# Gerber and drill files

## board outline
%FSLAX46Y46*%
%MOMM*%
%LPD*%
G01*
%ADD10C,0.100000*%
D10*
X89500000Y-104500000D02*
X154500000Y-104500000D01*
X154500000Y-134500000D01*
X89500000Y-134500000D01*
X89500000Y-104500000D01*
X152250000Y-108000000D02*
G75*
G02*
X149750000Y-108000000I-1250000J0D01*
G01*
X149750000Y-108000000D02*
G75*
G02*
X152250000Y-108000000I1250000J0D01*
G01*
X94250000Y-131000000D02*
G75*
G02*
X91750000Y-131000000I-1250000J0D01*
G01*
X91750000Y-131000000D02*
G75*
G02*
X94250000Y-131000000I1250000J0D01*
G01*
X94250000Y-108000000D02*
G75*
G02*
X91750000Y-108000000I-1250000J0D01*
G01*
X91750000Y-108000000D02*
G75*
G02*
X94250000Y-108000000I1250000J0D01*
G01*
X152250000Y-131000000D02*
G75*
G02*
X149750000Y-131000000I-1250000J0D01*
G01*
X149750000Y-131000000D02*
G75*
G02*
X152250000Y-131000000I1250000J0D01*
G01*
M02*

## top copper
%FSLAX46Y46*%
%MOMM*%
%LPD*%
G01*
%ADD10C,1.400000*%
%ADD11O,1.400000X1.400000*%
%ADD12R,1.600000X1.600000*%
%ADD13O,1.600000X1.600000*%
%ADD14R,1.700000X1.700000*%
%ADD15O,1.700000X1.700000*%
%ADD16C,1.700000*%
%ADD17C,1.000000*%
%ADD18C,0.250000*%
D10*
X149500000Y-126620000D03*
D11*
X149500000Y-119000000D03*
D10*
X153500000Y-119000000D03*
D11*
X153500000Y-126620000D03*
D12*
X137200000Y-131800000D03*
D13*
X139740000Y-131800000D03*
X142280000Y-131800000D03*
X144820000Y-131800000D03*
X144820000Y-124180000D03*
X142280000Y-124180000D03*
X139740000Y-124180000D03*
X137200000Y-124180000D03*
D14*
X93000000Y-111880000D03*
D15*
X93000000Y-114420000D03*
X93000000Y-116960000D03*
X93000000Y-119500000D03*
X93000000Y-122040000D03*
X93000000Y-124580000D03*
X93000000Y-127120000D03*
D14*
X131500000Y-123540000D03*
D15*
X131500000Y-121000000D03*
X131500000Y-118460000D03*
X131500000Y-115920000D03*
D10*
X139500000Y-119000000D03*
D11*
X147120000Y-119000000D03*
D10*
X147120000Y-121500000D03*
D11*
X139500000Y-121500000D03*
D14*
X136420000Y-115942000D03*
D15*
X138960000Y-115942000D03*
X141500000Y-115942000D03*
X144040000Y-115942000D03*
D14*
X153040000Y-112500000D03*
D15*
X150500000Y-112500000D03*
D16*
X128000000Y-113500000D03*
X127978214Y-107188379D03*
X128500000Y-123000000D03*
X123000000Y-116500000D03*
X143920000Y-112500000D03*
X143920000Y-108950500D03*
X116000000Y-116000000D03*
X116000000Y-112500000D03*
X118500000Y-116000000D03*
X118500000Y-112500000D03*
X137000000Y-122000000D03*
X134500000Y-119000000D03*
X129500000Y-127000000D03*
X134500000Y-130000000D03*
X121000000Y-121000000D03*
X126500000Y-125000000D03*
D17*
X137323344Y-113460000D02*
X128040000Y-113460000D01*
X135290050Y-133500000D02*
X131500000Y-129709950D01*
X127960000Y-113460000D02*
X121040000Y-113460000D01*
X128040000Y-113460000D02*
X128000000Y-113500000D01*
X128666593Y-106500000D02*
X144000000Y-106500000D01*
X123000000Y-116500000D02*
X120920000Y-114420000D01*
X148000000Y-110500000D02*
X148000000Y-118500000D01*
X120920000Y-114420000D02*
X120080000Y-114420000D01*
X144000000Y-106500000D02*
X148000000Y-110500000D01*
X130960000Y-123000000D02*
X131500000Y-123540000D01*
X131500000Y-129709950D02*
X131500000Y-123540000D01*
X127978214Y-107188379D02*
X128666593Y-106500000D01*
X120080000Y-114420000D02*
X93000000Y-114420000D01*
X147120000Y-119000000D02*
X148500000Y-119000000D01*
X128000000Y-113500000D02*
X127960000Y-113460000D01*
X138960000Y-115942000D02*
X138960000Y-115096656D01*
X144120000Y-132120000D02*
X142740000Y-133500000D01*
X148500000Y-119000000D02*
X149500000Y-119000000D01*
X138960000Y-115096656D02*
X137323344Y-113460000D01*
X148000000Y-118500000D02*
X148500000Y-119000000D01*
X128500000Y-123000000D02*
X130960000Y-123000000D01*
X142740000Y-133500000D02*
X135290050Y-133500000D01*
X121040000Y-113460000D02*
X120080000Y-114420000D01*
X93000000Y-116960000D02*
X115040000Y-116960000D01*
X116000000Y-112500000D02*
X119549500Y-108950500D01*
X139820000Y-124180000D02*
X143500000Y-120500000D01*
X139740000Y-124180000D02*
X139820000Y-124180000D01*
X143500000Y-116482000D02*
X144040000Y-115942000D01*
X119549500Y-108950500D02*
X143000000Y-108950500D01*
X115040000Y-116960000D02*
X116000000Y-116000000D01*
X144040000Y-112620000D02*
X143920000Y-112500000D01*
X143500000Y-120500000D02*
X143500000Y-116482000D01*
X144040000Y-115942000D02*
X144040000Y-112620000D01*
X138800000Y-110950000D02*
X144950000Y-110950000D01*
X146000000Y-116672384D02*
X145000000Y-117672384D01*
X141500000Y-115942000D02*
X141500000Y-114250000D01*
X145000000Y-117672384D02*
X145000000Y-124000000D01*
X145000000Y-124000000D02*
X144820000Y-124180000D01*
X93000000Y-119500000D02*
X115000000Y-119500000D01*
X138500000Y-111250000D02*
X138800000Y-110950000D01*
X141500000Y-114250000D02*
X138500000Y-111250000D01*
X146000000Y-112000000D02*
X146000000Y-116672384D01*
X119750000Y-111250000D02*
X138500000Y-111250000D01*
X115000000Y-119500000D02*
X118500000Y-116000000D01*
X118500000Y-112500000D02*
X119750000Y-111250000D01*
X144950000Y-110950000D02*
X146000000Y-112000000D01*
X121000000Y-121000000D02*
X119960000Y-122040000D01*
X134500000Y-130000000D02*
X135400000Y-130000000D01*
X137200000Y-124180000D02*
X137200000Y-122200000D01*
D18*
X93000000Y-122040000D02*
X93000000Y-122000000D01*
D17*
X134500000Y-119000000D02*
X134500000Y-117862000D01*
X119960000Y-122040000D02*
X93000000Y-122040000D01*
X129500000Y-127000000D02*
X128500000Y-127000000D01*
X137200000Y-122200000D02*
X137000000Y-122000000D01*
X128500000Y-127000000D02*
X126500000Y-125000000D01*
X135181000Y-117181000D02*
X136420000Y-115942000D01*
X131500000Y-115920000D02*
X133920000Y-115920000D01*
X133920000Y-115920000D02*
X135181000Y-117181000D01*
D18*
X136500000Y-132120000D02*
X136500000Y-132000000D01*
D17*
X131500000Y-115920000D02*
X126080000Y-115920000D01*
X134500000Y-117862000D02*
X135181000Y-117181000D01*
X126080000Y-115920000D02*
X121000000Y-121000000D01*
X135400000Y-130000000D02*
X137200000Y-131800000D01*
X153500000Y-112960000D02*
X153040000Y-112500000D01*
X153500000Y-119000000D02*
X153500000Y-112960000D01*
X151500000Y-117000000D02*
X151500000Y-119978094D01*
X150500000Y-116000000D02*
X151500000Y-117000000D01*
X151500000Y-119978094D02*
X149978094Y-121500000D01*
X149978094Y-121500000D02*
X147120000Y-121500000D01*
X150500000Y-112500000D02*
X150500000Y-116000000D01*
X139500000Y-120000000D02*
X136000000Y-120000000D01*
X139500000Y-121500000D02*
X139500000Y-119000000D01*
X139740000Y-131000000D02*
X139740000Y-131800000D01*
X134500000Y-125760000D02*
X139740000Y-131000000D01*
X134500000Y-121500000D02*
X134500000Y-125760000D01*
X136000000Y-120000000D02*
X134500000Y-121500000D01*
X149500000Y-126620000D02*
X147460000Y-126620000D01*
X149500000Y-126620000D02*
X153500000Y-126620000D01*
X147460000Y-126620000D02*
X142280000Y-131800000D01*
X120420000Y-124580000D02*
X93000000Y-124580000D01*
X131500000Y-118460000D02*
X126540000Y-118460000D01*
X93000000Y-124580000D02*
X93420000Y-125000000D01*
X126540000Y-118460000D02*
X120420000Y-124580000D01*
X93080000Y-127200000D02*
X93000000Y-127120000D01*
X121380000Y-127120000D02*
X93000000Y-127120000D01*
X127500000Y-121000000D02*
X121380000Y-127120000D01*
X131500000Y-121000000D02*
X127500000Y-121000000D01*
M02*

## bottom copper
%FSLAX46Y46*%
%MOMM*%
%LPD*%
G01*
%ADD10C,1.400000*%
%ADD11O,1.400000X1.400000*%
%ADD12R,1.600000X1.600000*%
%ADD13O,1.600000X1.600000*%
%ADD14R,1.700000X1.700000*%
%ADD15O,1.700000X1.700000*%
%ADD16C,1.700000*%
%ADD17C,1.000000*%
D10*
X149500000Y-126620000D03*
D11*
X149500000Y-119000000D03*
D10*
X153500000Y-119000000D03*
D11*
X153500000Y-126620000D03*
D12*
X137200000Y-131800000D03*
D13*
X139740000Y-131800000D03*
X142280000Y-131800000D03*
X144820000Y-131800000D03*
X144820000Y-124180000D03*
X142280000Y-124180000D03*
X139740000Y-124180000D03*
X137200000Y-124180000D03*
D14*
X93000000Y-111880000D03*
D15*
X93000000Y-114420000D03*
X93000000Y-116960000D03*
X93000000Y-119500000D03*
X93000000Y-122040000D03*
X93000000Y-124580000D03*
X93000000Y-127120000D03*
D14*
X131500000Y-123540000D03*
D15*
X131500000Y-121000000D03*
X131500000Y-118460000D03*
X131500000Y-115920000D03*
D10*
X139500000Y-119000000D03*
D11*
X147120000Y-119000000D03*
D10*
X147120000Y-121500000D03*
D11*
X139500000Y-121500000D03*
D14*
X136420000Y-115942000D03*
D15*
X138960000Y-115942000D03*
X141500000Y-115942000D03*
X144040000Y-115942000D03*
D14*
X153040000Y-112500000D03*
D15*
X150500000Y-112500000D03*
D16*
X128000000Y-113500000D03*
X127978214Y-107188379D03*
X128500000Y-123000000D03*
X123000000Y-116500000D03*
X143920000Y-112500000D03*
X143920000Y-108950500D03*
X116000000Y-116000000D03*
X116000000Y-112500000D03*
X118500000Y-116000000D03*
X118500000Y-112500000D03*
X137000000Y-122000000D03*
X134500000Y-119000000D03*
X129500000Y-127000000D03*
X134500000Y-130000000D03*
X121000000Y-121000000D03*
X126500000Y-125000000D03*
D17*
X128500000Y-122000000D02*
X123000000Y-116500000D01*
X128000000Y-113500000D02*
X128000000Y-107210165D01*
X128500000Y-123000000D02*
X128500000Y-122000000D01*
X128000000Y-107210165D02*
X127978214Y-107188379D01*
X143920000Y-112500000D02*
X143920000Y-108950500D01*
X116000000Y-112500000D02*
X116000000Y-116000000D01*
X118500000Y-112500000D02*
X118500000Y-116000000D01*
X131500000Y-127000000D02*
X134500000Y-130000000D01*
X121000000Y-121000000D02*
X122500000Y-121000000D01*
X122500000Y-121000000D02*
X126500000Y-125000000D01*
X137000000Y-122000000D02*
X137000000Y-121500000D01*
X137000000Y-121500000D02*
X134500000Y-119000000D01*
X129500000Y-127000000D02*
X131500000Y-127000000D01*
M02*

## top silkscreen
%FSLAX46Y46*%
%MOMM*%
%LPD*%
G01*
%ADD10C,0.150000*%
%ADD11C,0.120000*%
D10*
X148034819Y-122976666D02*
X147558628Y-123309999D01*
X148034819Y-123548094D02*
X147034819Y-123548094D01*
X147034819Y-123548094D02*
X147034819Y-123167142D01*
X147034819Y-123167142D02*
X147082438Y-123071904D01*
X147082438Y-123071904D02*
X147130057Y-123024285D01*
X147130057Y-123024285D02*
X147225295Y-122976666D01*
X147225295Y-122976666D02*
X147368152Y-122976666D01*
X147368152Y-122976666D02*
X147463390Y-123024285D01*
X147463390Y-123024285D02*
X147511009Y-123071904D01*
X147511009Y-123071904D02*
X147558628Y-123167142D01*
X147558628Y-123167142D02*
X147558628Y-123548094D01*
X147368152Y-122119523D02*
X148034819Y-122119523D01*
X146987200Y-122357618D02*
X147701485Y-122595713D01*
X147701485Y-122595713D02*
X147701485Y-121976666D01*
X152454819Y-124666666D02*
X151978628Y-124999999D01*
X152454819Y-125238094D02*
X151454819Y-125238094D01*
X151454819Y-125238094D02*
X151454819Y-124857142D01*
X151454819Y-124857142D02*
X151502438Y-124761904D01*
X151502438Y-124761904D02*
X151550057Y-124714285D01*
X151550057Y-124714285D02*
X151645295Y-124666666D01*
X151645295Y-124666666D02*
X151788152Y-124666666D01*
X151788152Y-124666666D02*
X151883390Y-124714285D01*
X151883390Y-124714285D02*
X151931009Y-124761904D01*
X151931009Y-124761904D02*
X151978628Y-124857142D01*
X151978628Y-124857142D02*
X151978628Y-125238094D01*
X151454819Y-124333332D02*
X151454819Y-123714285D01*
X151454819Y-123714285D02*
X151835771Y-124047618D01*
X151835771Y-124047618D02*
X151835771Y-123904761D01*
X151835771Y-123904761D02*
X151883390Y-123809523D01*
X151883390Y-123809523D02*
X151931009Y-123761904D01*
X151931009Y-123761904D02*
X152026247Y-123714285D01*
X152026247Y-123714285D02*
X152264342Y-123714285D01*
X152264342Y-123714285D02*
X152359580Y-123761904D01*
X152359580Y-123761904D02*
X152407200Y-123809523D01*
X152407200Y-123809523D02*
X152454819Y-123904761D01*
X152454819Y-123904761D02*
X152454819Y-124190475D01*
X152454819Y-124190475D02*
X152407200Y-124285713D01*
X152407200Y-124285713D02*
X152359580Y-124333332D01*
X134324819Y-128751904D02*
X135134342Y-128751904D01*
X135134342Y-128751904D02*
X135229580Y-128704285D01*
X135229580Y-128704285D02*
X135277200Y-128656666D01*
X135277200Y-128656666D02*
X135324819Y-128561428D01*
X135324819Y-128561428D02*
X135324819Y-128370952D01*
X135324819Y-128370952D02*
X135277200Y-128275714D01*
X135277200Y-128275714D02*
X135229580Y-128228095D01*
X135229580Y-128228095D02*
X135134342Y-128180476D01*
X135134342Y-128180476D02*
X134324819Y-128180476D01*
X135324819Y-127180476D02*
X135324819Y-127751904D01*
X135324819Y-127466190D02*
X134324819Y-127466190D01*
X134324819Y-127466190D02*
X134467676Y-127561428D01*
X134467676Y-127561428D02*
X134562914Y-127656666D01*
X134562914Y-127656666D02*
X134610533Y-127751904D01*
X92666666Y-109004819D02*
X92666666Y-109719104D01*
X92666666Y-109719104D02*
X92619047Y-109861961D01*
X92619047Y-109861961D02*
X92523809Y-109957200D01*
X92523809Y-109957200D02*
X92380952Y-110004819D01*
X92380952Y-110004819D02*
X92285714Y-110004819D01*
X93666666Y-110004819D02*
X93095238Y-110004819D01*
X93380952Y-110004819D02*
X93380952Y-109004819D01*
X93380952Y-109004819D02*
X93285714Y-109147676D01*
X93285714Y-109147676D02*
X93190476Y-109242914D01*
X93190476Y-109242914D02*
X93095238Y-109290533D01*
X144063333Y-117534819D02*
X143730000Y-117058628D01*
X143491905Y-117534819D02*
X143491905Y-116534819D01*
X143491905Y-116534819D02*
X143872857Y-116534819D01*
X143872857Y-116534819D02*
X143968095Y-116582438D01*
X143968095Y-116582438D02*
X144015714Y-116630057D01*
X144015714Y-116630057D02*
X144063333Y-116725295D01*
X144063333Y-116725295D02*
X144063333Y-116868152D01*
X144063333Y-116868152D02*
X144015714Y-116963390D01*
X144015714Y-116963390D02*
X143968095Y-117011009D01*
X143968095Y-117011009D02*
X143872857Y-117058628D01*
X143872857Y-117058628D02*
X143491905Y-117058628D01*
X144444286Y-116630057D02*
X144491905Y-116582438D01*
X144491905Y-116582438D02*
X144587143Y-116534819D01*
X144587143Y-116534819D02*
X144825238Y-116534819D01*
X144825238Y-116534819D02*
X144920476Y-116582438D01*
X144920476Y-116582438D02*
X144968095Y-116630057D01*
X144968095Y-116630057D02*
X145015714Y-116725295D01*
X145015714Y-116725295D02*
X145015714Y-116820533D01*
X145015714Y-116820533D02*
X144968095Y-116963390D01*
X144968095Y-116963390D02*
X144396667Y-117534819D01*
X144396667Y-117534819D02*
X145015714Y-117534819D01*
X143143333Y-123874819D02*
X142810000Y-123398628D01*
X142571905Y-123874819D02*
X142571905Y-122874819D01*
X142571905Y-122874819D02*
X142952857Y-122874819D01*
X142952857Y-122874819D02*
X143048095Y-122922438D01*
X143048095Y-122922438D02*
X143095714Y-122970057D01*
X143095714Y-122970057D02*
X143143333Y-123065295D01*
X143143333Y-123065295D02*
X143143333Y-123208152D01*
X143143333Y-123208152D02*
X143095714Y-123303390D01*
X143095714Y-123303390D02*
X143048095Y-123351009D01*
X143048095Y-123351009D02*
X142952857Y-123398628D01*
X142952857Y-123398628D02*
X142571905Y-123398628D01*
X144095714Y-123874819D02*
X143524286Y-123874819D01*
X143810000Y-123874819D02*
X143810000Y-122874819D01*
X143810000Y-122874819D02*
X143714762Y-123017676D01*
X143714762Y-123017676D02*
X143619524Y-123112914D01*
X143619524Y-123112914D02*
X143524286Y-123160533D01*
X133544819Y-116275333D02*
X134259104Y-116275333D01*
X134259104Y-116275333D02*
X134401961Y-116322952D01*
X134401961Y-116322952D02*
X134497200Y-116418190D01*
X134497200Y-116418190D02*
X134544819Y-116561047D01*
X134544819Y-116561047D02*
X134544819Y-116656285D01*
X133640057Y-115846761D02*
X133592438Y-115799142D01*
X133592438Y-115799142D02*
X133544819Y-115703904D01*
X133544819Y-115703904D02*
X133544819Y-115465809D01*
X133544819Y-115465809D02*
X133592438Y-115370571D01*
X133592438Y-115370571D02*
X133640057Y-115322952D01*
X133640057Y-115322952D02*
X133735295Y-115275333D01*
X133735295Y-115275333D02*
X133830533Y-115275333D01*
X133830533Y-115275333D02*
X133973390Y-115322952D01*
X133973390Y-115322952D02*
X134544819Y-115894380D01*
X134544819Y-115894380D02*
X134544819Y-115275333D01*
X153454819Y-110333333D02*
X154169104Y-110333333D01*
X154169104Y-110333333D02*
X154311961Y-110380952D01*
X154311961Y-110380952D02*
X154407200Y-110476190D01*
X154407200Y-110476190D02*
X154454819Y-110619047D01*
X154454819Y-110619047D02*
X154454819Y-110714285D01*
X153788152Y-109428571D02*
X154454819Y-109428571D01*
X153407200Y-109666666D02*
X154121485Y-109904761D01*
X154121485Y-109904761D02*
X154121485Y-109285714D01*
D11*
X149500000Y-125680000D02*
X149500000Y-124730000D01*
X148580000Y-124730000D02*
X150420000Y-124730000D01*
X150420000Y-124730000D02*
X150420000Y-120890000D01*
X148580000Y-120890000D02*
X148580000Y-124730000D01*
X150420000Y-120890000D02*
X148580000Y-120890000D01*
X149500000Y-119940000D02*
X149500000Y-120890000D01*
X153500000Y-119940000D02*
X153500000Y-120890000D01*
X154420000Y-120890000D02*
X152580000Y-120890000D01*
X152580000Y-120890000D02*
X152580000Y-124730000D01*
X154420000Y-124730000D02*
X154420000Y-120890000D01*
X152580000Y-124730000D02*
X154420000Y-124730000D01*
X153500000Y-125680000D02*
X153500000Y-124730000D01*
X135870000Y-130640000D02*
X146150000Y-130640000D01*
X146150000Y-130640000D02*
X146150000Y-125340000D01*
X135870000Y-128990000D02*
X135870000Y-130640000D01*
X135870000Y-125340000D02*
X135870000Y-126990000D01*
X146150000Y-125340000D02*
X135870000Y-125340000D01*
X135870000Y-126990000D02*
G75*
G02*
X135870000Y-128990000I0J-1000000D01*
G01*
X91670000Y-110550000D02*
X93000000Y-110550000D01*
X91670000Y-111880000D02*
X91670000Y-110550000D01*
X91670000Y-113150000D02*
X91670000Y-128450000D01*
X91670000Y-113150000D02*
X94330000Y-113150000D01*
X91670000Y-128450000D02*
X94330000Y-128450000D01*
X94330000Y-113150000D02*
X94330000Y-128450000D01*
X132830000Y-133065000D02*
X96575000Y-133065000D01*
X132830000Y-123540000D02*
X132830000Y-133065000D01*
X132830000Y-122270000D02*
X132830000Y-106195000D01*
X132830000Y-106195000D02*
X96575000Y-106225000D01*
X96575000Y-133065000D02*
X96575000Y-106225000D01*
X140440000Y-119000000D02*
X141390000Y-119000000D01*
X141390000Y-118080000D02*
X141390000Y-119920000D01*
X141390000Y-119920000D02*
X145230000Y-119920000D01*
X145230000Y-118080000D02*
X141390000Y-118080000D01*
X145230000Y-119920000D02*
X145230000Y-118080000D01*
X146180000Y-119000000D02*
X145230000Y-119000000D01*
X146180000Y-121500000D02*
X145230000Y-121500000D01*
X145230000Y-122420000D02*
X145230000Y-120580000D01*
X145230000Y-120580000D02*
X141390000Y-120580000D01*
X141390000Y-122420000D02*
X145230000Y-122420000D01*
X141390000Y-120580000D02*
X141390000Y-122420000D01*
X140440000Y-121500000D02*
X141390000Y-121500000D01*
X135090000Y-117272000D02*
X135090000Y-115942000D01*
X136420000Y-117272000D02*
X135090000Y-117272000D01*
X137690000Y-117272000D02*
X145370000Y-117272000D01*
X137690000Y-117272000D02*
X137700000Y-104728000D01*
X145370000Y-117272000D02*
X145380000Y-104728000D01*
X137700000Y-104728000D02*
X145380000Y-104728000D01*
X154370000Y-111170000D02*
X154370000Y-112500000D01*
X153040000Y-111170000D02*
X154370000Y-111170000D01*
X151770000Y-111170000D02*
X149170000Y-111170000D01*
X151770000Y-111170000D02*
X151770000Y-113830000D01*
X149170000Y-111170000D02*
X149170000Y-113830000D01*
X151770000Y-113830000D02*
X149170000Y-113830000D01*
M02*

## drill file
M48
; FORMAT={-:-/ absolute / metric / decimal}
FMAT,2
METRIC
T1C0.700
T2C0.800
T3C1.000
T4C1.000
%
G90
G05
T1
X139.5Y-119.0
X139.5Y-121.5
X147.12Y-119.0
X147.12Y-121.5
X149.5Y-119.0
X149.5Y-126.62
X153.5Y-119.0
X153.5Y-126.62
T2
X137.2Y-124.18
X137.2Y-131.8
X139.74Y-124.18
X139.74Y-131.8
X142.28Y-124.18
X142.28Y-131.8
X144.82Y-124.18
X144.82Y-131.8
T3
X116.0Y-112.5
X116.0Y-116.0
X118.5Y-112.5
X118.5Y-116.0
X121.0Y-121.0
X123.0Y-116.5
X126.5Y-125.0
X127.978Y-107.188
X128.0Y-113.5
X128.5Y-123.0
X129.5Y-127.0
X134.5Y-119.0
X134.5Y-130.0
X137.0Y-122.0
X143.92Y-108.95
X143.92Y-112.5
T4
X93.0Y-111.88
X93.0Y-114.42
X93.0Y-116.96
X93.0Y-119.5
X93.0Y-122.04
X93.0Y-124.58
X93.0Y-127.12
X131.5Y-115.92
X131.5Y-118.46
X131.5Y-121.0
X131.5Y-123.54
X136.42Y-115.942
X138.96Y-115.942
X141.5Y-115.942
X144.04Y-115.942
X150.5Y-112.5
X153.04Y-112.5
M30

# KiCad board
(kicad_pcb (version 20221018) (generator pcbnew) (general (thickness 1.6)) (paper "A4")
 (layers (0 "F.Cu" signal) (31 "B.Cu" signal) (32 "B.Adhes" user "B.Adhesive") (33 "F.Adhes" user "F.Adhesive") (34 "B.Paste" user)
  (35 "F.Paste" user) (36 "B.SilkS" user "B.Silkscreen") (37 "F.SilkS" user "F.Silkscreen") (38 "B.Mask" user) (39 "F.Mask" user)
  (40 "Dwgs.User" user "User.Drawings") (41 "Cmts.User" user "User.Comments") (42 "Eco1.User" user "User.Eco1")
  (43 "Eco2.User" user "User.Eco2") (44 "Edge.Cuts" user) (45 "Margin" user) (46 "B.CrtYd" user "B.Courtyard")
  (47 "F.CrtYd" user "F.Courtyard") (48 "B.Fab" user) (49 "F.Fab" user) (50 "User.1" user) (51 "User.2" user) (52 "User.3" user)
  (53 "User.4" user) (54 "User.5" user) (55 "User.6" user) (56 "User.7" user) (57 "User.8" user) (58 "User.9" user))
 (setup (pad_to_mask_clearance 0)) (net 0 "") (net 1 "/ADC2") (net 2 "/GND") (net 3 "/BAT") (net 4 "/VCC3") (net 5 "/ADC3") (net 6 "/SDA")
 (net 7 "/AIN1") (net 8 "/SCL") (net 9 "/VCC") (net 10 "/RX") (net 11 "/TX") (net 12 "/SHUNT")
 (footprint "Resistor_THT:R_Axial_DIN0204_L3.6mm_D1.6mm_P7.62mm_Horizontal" (layer "F.Cu") (at 149.5 126.62 90)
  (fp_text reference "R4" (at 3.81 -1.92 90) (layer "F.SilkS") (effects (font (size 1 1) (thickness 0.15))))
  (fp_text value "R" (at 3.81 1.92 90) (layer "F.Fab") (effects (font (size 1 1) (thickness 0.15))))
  (fp_line (start 0.94 0) (end 1.89 0) (stroke (width 0.12) (type solid)) (layer "F.SilkS"))
  (fp_line (start 1.89 -0.92) (end 1.89 0.92) (stroke (width 0.12) (type solid)) (layer "F.SilkS"))
  (fp_line (start 1.89 0.92) (end 5.73 0.92) (stroke (width 0.12) (type solid)) (layer "F.SilkS"))
  (fp_line (start 5.73 -0.92) (end 1.89 -0.92) (stroke (width 0.12) (type solid)) (layer "F.SilkS"))
  (fp_line (start 5.73 0.92) (end 5.73 -0.92) (stroke (width 0.12) (type solid)) (layer "F.SilkS"))
  (fp_line (start 6.68 0) (end 5.73 0) (stroke (width 0.12) (type solid)) (layer "F.SilkS"))
  (pad "1" thru_hole circle (at 0 0 90) (size 1.4 1.4) (drill 0.7) (layers "*.Cu" "*.Mask") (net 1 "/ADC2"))
  (pad "2" thru_hole oval (at 7.62 0 90) (size 1.4 1.4) (drill 0.7) (layers "*.Cu" "*.Mask") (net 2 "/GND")))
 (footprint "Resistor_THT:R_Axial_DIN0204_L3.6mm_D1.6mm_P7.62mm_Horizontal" (layer "F.Cu") (at 153.5 119 -90)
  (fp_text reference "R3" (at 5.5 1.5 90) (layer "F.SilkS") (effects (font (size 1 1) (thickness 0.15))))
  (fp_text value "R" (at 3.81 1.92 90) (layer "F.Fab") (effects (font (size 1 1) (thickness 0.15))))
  (fp_line (start 0.94 0) (end 1.89 0) (stroke (width 0.12) (type solid)) (layer "F.SilkS"))
  (fp_line (start 1.89 -0.92) (end 1.89 0.92) (stroke (width 0.12) (type solid)) (layer "F.SilkS"))
  (fp_line (start 1.89 0.92) (end 5.73 0.92) (stroke (width 0.12) (type solid)) (layer "F.SilkS"))
  (fp_line (start 5.73 -0.92) (end 1.89 -0.92) (stroke (width 0.12) (type solid)) (layer "F.SilkS"))
  (fp_line (start 5.73 0.92) (end 5.73 -0.92) (stroke (width 0.12) (type solid)) (layer "F.SilkS"))
  (fp_line (start 6.68 0) (end 5.73 0) (stroke (width 0.12) (type solid)) (layer "F.SilkS"))
  (pad "1" thru_hole circle (at 0 0 270) (size 1.4 1.4) (drill 0.7) (layers "*.Cu" "*.Mask") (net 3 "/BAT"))
  (pad "2" thru_hole oval (at 7.62 0 270) (size 1.4 1.4) (drill 0.7) (layers "*.Cu" "*.Mask") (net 1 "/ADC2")))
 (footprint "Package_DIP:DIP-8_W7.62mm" (layer "F.Cu") (at 137.2 131.8 90)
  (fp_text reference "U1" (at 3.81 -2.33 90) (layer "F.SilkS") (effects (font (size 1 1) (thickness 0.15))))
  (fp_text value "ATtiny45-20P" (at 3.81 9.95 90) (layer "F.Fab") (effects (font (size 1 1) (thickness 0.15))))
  (fp_line (start 1.16 -1.33) (end 1.16 8.95) (stroke (width 0.12) (type solid)) (layer "F.SilkS"))
  (fp_line (start 1.16 8.95) (end 6.46 8.95) (stroke (width 0.12) (type solid)) (layer "F.SilkS"))
  (fp_line (start 2.81 -1.33) (end 1.16 -1.33) (stroke (width 0.12) (type solid)) (layer "F.SilkS"))
  (fp_line (start 6.46 -1.33) (end 4.81 -1.33) (stroke (width 0.12) (type solid)) (layer "F.SilkS"))
  (fp_line (start 6.46 8.95) (end 6.46 -1.33) (stroke (width 0.12) (type solid)) (layer "F.SilkS"))
  (fp_arc (start 4.81 -1.33) (mid 3.81 -0.33) (end 2.81 -1.33) (stroke (width 0.12) (type solid)) (layer "F.SilkS"))
  (pad "1" thru_hole rect (at 0 0 90) (size 1.6 1.6) (drill 0.8) (layers "*.Cu" "*.Mask") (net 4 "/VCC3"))
  (pad "2" thru_hole oval (at 0 2.54 90) (size 1.6 1.6) (drill 0.8) (layers "*.Cu" "*.Mask") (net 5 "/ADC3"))
  (pad "3" thru_hole oval (at 0 5.08 90) (size 1.6 1.6) (drill 0.8) (layers "*.Cu" "*.Mask") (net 1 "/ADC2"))
  (pad "4" thru_hole oval (at 0 7.62 90) (size 1.6 1.6) (drill 0.8) (layers "*.Cu" "*.Mask") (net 2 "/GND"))
  (pad "5" thru_hole oval (at 7.62 7.62 90) (size 1.6 1.6) (drill 0.8) (layers "*.Cu" "*.Mask") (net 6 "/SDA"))
  (pad "6" thru_hole oval (at 7.62 5.08 90) (size 1.6 1.6) (drill 0.8) (layers "*.Cu" "*.Mask") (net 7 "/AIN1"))
  (pad "7" thru_hole oval (at 7.62 2.54 90) (size 1.6 1.6) (drill 0.8) (layers "*.Cu" "*.Mask") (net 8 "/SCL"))
  (pad "8" thru_hole oval (at 7.62 0 90) (size 1.6 1.6) (drill 0.8) (layers "*.Cu" "*.Mask") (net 4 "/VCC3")))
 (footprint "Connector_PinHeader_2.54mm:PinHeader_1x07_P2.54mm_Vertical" (layer "F.Cu") (at 93 111.88)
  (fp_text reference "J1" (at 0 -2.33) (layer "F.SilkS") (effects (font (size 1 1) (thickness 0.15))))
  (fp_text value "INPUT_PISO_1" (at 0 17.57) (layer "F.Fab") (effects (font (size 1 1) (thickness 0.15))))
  (fp_line (start -1.33 -1.33) (end 0 -1.33) (stroke (width 0.12) (type solid)) (layer "F.SilkS"))
  (fp_line (start -1.33 0) (end -1.33 -1.33) (stroke (width 0.12) (type solid)) (layer "F.SilkS"))
  (fp_line (start -1.33 1.27) (end -1.33 16.57) (stroke (width 0.12) (type solid)) (layer "F.SilkS"))
  (fp_line (start -1.33 1.27) (end 1.33 1.27) (stroke (width 0.12) (type solid)) (layer "F.SilkS"))
  (fp_line (start -1.33 16.57) (end 1.33 16.57) (stroke (width 0.12) (type solid)) (layer "F.SilkS"))
  (fp_line (start 1.33 1.27) (end 1.33 16.57) (stroke (width 0.12) (type solid)) (layer "F.SilkS"))
  (pad "1" thru_hole rect (at 0 0) (size 1.7 1.7) (drill 1) (layers "*.Cu" "*.Mask") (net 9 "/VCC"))
  (pad "2" thru_hole oval (at 0 2.54) (size 1.7 1.7) (drill 1) (layers "*.Cu" "*.Mask") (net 2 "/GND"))
  (pad "3" thru_hole oval (at 0 5.08) (size 1.7 1.7) (drill 1) (layers "*.Cu" "*.Mask") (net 8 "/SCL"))
  (pad "4" thru_hole oval (at 0 7.62) (size 1.7 1.7) (drill 1) (layers "*.Cu" "*.Mask") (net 6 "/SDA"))
  (pad "5" thru_hole oval (at 0 10.16) (size 1.7 1.7) (drill 1) (layers "*.Cu" "*.Mask") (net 4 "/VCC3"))
  (pad "6" thru_hole oval (at 0 12.7) (size 1.7 1.7) (drill 1) (layers "*.Cu" "*.Mask") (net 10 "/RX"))
  (pad "7" thru_hole oval (at 0 15.24) (size 1.7 1.7) (drill 1) (layers "*.Cu" "*.Mask") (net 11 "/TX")))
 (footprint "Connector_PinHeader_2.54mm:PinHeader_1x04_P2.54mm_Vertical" (layer "F.Cu") (at 131.5 123.54 180)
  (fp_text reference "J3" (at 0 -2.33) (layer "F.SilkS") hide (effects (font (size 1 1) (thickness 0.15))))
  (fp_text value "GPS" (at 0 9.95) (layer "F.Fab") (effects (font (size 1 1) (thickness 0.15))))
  (fp_line (start -1.33 -9.525) (end 34.925 -9.525) (stroke (width 0.12) (type solid)) (layer "F.SilkS"))
  (fp_line (start -1.33 0) (end -1.33 -9.525) (stroke (width 0.12) (type solid)) (layer "F.SilkS"))
  (fp_line (start -1.33 1.27) (end -1.33 17.345) (stroke (width 0.12) (type solid)) (layer "F.SilkS"))
  (fp_line (start -1.33 17.345) (end 34.925 17.315) (stroke (width 0.12) (type solid)) (layer "F.SilkS"))
  (fp_line (start 34.925 -9.525) (end 34.925 17.315) (stroke (width 0.12) (type solid)) (layer "F.SilkS"))
  (pad "1" thru_hole rect (at 0 0 180) (size 1.7 1.7) (drill 1) (layers "*.Cu" "*.Mask") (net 2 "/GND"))
  (pad "2" thru_hole oval (at 0 2.54 180) (size 1.7 1.7) (drill 1) (layers "*.Cu" "*.Mask") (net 11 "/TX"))
  (pad "3" thru_hole oval (at 0 5.08 180) (size 1.7 1.7) (drill 1) (layers "*.Cu" "*.Mask") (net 10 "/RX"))
  (pad "4" thru_hole oval (at 0 7.62 180) (size 1.7 1.7) (drill 1) (layers "*.Cu" "*.Mask") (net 4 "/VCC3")))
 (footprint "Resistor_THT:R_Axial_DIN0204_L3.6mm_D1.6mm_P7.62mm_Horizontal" (layer "F.Cu") (at 139.5 119)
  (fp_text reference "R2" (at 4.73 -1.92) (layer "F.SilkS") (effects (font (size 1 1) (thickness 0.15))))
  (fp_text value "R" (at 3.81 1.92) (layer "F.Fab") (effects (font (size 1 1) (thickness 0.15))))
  (fp_line (start 0.94 0) (end 1.89 0) (stroke (width 0.12) (type solid)) (layer "F.SilkS"))
  (fp_line (start 1.89 -0.92) (end 1.89 0.92) (stroke (width 0.12) (type solid)) (layer "F.SilkS"))
  (fp_line (start 1.89 0.92) (end 5.73 0.92) (stroke (width 0.12) (type solid)) (layer "F.SilkS"))
  (fp_line (start 5.73 -0.92) (end 1.89 -0.92) (stroke (width 0.12) (type solid)) (layer "F.SilkS"))
  (fp_line (start 5.73 0.92) (end 5.73 -0.92) (stroke (width 0.12) (type solid)) (layer "F.SilkS"))
  (fp_line (start 6.68 0) (end 5.73 0) (stroke (width 0.12) (type solid)) (layer "F.SilkS"))
  (pad "1" thru_hole circle (at 0 0) (size 1.4 1.4) (drill 0.7) (layers "*.Cu" "*.Mask") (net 5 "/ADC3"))
  (pad "2" thru_hole oval (at 7.62 0) (size 1.4 1.4) (drill 0.7) (layers "*.Cu" "*.Mask") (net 2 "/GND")))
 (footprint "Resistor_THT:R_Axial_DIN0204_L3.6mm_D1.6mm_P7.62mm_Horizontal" (layer "F.Cu") (at 147.12 121.5 180)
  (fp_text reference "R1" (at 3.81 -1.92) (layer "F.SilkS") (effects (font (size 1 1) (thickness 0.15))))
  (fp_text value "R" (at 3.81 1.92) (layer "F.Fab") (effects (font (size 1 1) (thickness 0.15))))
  (fp_line (start 0.94 0) (end 1.89 0) (stroke (width 0.12) (type solid)) (layer "F.SilkS"))
  (fp_line (start 1.89 -0.92) (end 1.89 0.92) (stroke (width 0.12) (type solid)) (layer "F.SilkS"))
  (fp_line (start 1.89 0.92) (end 5.73 0.92) (stroke (width 0.12) (type solid)) (layer "F.SilkS"))
  (fp_line (start 5.73 -0.92) (end 1.89 -0.92) (stroke (width 0.12) (type solid)) (layer "F.SilkS"))
  (fp_line (start 5.73 0.92) (end 5.73 -0.92) (stroke (width 0.12) (type solid)) (layer "F.SilkS"))
  (fp_line (start 6.68 0) (end 5.73 0) (stroke (width 0.12) (type solid)) (layer "F.SilkS"))
  (pad "1" thru_hole circle (at 0 0 180) (size 1.4 1.4) (drill 0.7) (layers "*.Cu" "*.Mask") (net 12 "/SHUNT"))
  (pad "2" thru_hole oval (at 7.62 0 180) (size 1.4 1.4) (drill 0.7) (layers "*.Cu" "*.Mask") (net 5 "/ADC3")))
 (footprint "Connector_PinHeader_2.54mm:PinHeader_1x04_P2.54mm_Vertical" (layer "F.Cu") (at 136.42 115.942 90)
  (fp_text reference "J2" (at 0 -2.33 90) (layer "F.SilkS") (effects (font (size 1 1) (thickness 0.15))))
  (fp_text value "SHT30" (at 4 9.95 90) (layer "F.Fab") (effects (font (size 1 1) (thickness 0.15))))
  (fp_line (start -1.33 -1.33) (end 0 -1.33) (stroke (width 0.12) (type solid)) (layer "F.SilkS"))
  (fp_line (start -1.33 0) (end -1.33 -1.33) (stroke (width 0.12) (type solid)) (layer "F.SilkS"))
  (fp_line (start -1.33 1.27) (end -1.33 8.95) (stroke (width 0.12) (type solid)) (layer "F.SilkS"))
  (fp_line (start -1.33 1.27) (end 11.214 1.28) (stroke (width 0.12) (type solid)) (layer "F.SilkS"))
  (fp_line (start -1.33 8.95) (end 11.214 8.96) (stroke (width 0.12) (type solid)) (layer "F.SilkS"))
  (fp_line (start 11.214 1.28) (end 11.214 8.96) (stroke (width 0.12) (type solid)) (layer "F.SilkS"))
  (pad "1" thru_hole rect (at 0 0 90) (size 1.7 1.7) (drill 1) (layers "*.Cu" "*.Mask") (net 4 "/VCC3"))
  (pad "2" thru_hole oval (at 0 2.54 90) (size 1.7 1.7) (drill 1) (layers "*.Cu" "*.Mask") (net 2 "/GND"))
  (pad "3" thru_hole oval (at 0 5.08 90) (size 1.7 1.7) (drill 1) (layers "*.Cu" "*.Mask") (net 6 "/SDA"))
  (pad "4" thru_hole oval (at 0 7.62 90) (size 1.7 1.7) (drill 1) (layers "*.Cu" "*.Mask") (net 8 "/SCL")))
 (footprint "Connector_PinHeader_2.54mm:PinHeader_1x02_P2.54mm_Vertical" (layer "F.Cu") (at 153.04 112.5 -90)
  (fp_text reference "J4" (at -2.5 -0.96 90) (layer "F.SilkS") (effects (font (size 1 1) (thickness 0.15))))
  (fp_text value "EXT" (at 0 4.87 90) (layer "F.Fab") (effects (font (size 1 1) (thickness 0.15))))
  (fp_line (start -1.33 -1.33) (end 0 -1.33) (stroke (width 0.12) (type solid)) (layer "F.SilkS"))
  (fp_line (start -1.33 0) (end -1.33 -1.33) (stroke (width 0.12) (type solid)) (layer "F.SilkS"))
  (fp_line (start -1.33 1.27) (end -1.33 3.87) (stroke (width 0.12) (type solid)) (layer "F.SilkS"))
  (fp_line (start -1.33 1.27) (end 1.33 1.27) (stroke (width 0.12) (type solid)) (layer "F.SilkS"))
  (fp_line (start -1.33 3.87) (end 1.33 3.87) (stroke (width 0.12) (type solid)) (layer "F.SilkS"))
  (fp_line (start 1.33 1.27) (end 1.33 3.87) (stroke (width 0.12) (type solid)) (layer "F.SilkS"))
  (pad "1" thru_hole rect (at 0 0 270) (size 1.7 1.7) (drill 1) (layers "*.Cu" "*.Mask") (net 3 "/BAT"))
  (pad "2" thru_hole oval (at 0 2.54 270) (size 1.7 1.7) (drill 1) (layers "*.Cu" "*.Mask") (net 12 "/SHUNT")))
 (gr_rect (start 89.5 104.5) (end 154.5 134.5) (stroke (width 0.1) (type default)) (fill none) (layer "Edge.Cuts"))
 (gr_circle (center 151 108) (end 152.25 108) (stroke (width 0.1) (type default)) (fill none) (layer "Edge.Cuts"))
 (gr_circle (center 93 131) (end 94.25 131) (stroke (width 0.1) (type default)) (fill none) (layer "Edge.Cuts"))
 (gr_circle (center 93 108) (end 94.25 108) (stroke (width 0.1) (type default)) (fill none) (layer "Edge.Cuts"))
 (gr_circle (center 151 131) (end 152.25 131) (stroke (width 0.1) (type default)) (fill none) (layer "Edge.Cuts"))
 (segment (start 137.323344 113.46) (end 128.04 113.46) (width 1) (layer "F.Cu") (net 2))
 (segment (start 135.29005 133.5) (end 131.5 129.70995) (width 1) (layer "F.Cu") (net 2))
 (segment (start 127.96 113.46) (end 121.04 113.46) (width 1) (layer "F.Cu") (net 2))
 (segment (start 128.04 113.46) (end 128 113.5) (width 1) (layer "F.Cu") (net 2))
 (segment (start 128.666593 106.5) (end 144 106.5) (width 1) (layer "F.Cu") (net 2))
 (segment (start 123 116.5) (end 120.92 114.42) (width 1) (layer "F.Cu") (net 2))
 (segment (start 148 110.5) (end 148 118.5) (width 1) (layer "F.Cu") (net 2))
 (segment (start 120.92 114.42) (end 120.08 114.42) (width 1) (layer "F.Cu") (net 2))
 (segment (start 144 106.5) (end 148 110.5) (width 1) (layer "F.Cu") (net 2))
 (segment (start 130.96 123) (end 131.5 123.54) (width 1) (layer "F.Cu") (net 2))
 (segment (start 131.5 129.70995) (end 131.5 123.54) (width 1) (layer "F.Cu") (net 2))
 (segment (start 127.978214 107.188379) (end 128.666593 106.5) (width 1) (layer "F.Cu") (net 2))
 (segment (start 120.08 114.42) (end 93 114.42) (width 1) (layer "F.Cu") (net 2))
 (segment (start 147.12 119) (end 148.5 119) (width 1) (layer "F.Cu") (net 2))
 (segment (start 128 113.5) (end 127.96 113.46) (width 1) (layer "F.Cu") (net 2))
 (segment (start 138.96 115.942) (end 138.96 115.096656) (width 1) (layer "F.Cu") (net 2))
 (segment (start 144.12 132.12) (end 142.74 133.5) (width 1) (layer "F.Cu") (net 2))
 (segment (start 148.5 119) (end 149.5 119) (width 1) (layer "F.Cu") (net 2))
 (segment (start 138.96 115.096656) (end 137.323344 113.46) (width 1) (layer "F.Cu") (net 2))
 (segment (start 148 118.5) (end 148.5 119) (width 1) (layer "F.Cu") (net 2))
 (segment (start 128.5 123) (end 130.96 123) (width 1) (layer "F.Cu") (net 2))
 (segment (start 142.74 133.5) (end 135.29005 133.5) (width 1) (layer "F.Cu") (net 2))
 (segment (start 121.04 113.46) (end 120.08 114.42) (width 1) (layer "F.Cu") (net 2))
 (via (at 128 113.5) (size 1.7) (drill 1) (layers "F.Cu" "B.Cu") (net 2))
 (via (at 127.978214 107.188379) (size 1.7) (drill 1) (layers "F.Cu" "B.Cu") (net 2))
 (via (at 128.5 123) (size 1.7) (drill 1) (layers "F.Cu" "B.Cu") (free) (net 2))
 (via (at 123 116.5) (size 1.7) (drill 1) (layers "F.Cu" "B.Cu") (free) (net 2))
 (segment (start 128.5 122) (end 123 116.5) (width 1) (layer "B.Cu") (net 2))
 (segment (start 128 113.5) (end 128 107.210165) (width 1) (layer "B.Cu") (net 2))
 (segment (start 128.5 123) (end 128.5 122) (width 1) (layer "B.Cu") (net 2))
 (segment (start 128 107.210165) (end 127.978214 107.188379) (width 1) (layer "B.Cu") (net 2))
 (segment (start 93 116.96) (end 115.04 116.96) (width 1) (layer "F.Cu") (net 8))
 (segment (start 116 112.5) (end 119.5495 108.9505) (width 1) (layer "F.Cu") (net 8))
 (segment (start 139.82 124.18) (end 143.5 120.5) (width 1) (layer "F.Cu") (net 8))
 (segment (start 139.74 124.18) (end 139.82 124.18) (width 1) (layer "F.Cu") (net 8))
 (segment (start 143.5 116.482) (end 144.04 115.942) (width 1) (layer "F.Cu") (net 8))
 (segment (start 119.5495 108.9505) (end 143 108.9505) (width 1) (layer "F.Cu") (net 8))
 (segment (start 115.04 116.96) (end 116 116) (width 1) (layer "F.Cu") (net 8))
 (segment (start 144.04 112.62) (end 143.92 112.5) (width 1) (layer "F.Cu") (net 8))
 (segment (start 143.5 120.5) (end 143.5 116.482) (width 1) (layer "F.Cu") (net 8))
 (segment (start 144.04 115.942) (end 144.04 112.62) (width 1) (layer "F.Cu") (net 8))
 (via (at 143.92 112.5) (size 1.7) (drill 1) (layers "F.Cu" "B.Cu") (free) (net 8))
 (via (at 143.92 108.9505) (size 1.7) (drill 1) (layers "F.Cu" "B.Cu") (free) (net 8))
 (via (at 116 116) (size 1.7) (drill 1) (layers "F.Cu" "B.Cu") (free) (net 8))
 (via (at 116 112.5) (size 1.7) (drill 1) (layers "F.Cu" "B.Cu") (free) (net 8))
 (segment (start 143.92 112.5) (end 143.92 108.9505) (width 1) (layer "B.Cu") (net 8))
 (segment (start 116 112.5) (end 116 116) (width 1) (layer "B.Cu") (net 8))
 (segment (start 138.8 110.95) (end 144.95 110.95) (width 1) (layer "F.Cu") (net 6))
 (segment (start 146 116.672384) (end 145 117.672384) (width 1) (layer "F.Cu") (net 6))
 (segment (start 141.5 115.942) (end 141.5 114.25) (width 1) (layer "F.Cu") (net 6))
 (segment (start 145 117.672384) (end 145 124) (width 1) (layer "F.Cu") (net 6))
 (segment (start 145 124) (end 144.82 124.18) (width 1) (layer "F.Cu") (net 6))
 (segment (start 93 119.5) (end 115 119.5) (width 1) (layer "F.Cu") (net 6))
 (segment (start 138.5 111.25) (end 138.8 110.95) (width 1) (layer "F.Cu") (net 6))
 (segment (start 141.5 114.25) (end 138.5 111.25) (width 1) (layer "F.Cu") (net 6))
 (segment (start 146 112) (end 146 116.672384) (width 1) (layer "F.Cu") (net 6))
 (segment (start 119.75 111.25) (end 138.5 111.25) (width 1) (layer "F.Cu") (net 6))
 (segment (start 115 119.5) (end 118.5 116) (width 1) (layer "F.Cu") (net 6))
 (segment (start 118.5 112.5) (end 119.75 111.25) (width 1) (layer "F.Cu") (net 6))
 (segment (start 144.95 110.95) (end 146 112) (width 1) (layer "F.Cu") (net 6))
 (via (at 118.5 116) (size 1.7) (drill 1) (layers "F.Cu" "B.Cu") (free) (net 6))
 (via (at 118.5 112.5) (size 1.7) (drill 1) (layers "F.Cu" "B.Cu") (free) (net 6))
 (segment (start 118.5 112.5) (end 118.5 116) (width 1) (layer "B.Cu") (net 6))
 (segment (start 121 121) (end 119.96 122.04) (width 1) (layer "F.Cu") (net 4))
 (segment (start 134.5 130) (end 135.4 130) (width 1) (layer "F.Cu") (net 4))
 (segment (start 137.2 124.18) (end 137.2 122.2) (width 1) (layer "F.Cu") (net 4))
 (segment (start 93 122.04) (end 93 122) (width 0.25) (layer "F.Cu") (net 4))
 (segment (start 134.5 119) (end 134.5 117.862) (width 1) (layer "F.Cu") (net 4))
 (segment (start 119.96 122.04) (end 93 122.04) (width 1) (layer "F.Cu") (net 4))
 (segment (start 129.5 127) (end 128.5 127) (width 1) (layer "F.Cu") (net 4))
 (segment (start 137.2 122.2) (end 137 122) (width 1) (layer "F.Cu") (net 4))
 (segment (start 128.5 127) (end 126.5 125) (width 1) (layer "F.Cu") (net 4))
 (segment (start 135.181 117.181) (end 136.42 115.942) (width 1) (layer "F.Cu") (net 4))
 (segment (start 131.5 115.92) (end 133.92 115.92) (width 1) (layer "F.Cu") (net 4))
 (segment (start 133.92 115.92) (end 135.181 117.181) (width 1) (layer "F.Cu") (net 4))
 (segment (start 136.5 132.12) (end 136.5 132) (width 0.25) (layer "F.Cu") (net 4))
 (segment (start 131.5 115.92) (end 126.08 115.92) (width 1) (layer "F.Cu") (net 4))
 (segment (start 134.5 117.862) (end 135.181 117.181) (width 1) (layer "F.Cu") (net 4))
 (segment (start 126.08 115.92) (end 121 121) (width 1) (layer "F.Cu") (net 4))
 (segment (start 135.4 130) (end 137.2 131.8) (width 1) (layer "F.Cu") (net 4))
 (via (at 137 122) (size 1.7) (drill 1) (layers "F.Cu" "B.Cu") (free) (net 4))
 (via (at 134.5 119) (size 1.7) (drill 1) (layers "F.Cu" "B.Cu") (free) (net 4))
 (via (at 129.5 127) (size 1.7) (drill 1) (layers "F.Cu" "B.Cu") (free) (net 4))
 (via (at 134.5 130) (size 1.7) (drill 1) (layers "F.Cu" "B.Cu") (free) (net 4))
 (via (at 121 121) (size 1.7) (drill 1) (layers "F.Cu" "B.Cu") (free) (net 4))
 (via (at 126.5 125) (size 1.7) (drill 1) (layers "F.Cu" "B.Cu") (free) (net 4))
 (segment (start 131.5 127) (end 134.5 130) (width 1) (layer "B.Cu") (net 4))
 (segment (start 121 121) (end 122.5 121) (width 1) (layer "B.Cu") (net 4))
 (segment (start 122.5 121) (end 126.5 125) (width 1) (layer "B.Cu") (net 4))
 (segment (start 137 122) (end 137 121.5) (width 1) (layer "B.Cu") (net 4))
 (segment (start 137 121.5) (end 134.5 119) (width 1) (layer "B.Cu") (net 4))
 (segment (start 129.5 127) (end 131.5 127) (width 1) (layer "B.Cu") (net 4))
 (segment (start 153.5 112.96) (end 153.04 112.5) (width 1) (layer "F.Cu") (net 3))
 (segment (start 153.5 119) (end 153.5 112.96) (width 1) (layer "F.Cu") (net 3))
 (segment (start 151.5 117) (end 151.5 119.978094) (width 1) (layer "F.Cu") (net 12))
 (segment (start 150.5 116) (end 151.5 117) (width 1) (layer "F.Cu") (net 12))
 (segment (start 151.5 119.978094) (end 149.978094 121.5) (width 1) (layer "F.Cu") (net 12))
 (segment (start 149.978094 121.5) (end 147.12 121.5) (width 1) (layer "F.Cu") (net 12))
 (segment (start 150.5 112.5) (end 150.5 116) (width 1) (layer "F.Cu") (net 12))
 (segment (start 139.5 120) (end 136 120) (width 1) (layer "F.Cu") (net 5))
 (segment (start 139.5 121.5) (end 139.5 119) (width 1) (layer "F.Cu") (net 5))
 (segment (start 139.74 131) (end 139.74 131.8) (width 1) (layer "F.Cu") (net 5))
 (segment (start 134.5 125.76) (end 139.74 131) (width 1) (layer "F.Cu") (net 5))
 (segment (start 134.5 121.5) (end 134.5 125.76) (width 1) (layer "F.Cu") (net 5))
 (segment (start 136 120) (end 134.5 121.5) (width 1) (layer "F.Cu") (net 5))
 (segment (start 149.5 126.62) (end 147.46 126.62) (width 1) (layer "F.Cu") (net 1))
 (segment (start 149.5 126.62) (end 153.5 126.62) (width 1) (layer "F.Cu") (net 1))
 (segment (start 147.46 126.62) (end 142.28 131.8) (width 1) (layer "F.Cu") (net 1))
 (segment (start 120.42 124.58) (end 93 124.58) (width 1) (layer "F.Cu") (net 10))
 (segment (start 131.5 118.46) (end 126.54 118.46) (width 1) (layer "F.Cu") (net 10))
 (segment (start 93 124.58) (end 93.42 125) (width 1) (layer "F.Cu") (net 10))
 (segment (start 126.54 118.46) (end 120.42 124.58) (width 1) (layer "F.Cu") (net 10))
 (segment (start 93.08 127.2) (end 93 127.12) (width 1) (layer "F.Cu") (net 11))
 (segment (start 121.38 127.12) (end 93 127.12) (width 1) (layer "F.Cu") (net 11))
 (segment (start 127.5 121) (end 121.38 127.12) (width 1) (layer "F.Cu") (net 11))
 (segment (start 131.5 121) (end 127.5 121) (width 1) (layer "F.Cu") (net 11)))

